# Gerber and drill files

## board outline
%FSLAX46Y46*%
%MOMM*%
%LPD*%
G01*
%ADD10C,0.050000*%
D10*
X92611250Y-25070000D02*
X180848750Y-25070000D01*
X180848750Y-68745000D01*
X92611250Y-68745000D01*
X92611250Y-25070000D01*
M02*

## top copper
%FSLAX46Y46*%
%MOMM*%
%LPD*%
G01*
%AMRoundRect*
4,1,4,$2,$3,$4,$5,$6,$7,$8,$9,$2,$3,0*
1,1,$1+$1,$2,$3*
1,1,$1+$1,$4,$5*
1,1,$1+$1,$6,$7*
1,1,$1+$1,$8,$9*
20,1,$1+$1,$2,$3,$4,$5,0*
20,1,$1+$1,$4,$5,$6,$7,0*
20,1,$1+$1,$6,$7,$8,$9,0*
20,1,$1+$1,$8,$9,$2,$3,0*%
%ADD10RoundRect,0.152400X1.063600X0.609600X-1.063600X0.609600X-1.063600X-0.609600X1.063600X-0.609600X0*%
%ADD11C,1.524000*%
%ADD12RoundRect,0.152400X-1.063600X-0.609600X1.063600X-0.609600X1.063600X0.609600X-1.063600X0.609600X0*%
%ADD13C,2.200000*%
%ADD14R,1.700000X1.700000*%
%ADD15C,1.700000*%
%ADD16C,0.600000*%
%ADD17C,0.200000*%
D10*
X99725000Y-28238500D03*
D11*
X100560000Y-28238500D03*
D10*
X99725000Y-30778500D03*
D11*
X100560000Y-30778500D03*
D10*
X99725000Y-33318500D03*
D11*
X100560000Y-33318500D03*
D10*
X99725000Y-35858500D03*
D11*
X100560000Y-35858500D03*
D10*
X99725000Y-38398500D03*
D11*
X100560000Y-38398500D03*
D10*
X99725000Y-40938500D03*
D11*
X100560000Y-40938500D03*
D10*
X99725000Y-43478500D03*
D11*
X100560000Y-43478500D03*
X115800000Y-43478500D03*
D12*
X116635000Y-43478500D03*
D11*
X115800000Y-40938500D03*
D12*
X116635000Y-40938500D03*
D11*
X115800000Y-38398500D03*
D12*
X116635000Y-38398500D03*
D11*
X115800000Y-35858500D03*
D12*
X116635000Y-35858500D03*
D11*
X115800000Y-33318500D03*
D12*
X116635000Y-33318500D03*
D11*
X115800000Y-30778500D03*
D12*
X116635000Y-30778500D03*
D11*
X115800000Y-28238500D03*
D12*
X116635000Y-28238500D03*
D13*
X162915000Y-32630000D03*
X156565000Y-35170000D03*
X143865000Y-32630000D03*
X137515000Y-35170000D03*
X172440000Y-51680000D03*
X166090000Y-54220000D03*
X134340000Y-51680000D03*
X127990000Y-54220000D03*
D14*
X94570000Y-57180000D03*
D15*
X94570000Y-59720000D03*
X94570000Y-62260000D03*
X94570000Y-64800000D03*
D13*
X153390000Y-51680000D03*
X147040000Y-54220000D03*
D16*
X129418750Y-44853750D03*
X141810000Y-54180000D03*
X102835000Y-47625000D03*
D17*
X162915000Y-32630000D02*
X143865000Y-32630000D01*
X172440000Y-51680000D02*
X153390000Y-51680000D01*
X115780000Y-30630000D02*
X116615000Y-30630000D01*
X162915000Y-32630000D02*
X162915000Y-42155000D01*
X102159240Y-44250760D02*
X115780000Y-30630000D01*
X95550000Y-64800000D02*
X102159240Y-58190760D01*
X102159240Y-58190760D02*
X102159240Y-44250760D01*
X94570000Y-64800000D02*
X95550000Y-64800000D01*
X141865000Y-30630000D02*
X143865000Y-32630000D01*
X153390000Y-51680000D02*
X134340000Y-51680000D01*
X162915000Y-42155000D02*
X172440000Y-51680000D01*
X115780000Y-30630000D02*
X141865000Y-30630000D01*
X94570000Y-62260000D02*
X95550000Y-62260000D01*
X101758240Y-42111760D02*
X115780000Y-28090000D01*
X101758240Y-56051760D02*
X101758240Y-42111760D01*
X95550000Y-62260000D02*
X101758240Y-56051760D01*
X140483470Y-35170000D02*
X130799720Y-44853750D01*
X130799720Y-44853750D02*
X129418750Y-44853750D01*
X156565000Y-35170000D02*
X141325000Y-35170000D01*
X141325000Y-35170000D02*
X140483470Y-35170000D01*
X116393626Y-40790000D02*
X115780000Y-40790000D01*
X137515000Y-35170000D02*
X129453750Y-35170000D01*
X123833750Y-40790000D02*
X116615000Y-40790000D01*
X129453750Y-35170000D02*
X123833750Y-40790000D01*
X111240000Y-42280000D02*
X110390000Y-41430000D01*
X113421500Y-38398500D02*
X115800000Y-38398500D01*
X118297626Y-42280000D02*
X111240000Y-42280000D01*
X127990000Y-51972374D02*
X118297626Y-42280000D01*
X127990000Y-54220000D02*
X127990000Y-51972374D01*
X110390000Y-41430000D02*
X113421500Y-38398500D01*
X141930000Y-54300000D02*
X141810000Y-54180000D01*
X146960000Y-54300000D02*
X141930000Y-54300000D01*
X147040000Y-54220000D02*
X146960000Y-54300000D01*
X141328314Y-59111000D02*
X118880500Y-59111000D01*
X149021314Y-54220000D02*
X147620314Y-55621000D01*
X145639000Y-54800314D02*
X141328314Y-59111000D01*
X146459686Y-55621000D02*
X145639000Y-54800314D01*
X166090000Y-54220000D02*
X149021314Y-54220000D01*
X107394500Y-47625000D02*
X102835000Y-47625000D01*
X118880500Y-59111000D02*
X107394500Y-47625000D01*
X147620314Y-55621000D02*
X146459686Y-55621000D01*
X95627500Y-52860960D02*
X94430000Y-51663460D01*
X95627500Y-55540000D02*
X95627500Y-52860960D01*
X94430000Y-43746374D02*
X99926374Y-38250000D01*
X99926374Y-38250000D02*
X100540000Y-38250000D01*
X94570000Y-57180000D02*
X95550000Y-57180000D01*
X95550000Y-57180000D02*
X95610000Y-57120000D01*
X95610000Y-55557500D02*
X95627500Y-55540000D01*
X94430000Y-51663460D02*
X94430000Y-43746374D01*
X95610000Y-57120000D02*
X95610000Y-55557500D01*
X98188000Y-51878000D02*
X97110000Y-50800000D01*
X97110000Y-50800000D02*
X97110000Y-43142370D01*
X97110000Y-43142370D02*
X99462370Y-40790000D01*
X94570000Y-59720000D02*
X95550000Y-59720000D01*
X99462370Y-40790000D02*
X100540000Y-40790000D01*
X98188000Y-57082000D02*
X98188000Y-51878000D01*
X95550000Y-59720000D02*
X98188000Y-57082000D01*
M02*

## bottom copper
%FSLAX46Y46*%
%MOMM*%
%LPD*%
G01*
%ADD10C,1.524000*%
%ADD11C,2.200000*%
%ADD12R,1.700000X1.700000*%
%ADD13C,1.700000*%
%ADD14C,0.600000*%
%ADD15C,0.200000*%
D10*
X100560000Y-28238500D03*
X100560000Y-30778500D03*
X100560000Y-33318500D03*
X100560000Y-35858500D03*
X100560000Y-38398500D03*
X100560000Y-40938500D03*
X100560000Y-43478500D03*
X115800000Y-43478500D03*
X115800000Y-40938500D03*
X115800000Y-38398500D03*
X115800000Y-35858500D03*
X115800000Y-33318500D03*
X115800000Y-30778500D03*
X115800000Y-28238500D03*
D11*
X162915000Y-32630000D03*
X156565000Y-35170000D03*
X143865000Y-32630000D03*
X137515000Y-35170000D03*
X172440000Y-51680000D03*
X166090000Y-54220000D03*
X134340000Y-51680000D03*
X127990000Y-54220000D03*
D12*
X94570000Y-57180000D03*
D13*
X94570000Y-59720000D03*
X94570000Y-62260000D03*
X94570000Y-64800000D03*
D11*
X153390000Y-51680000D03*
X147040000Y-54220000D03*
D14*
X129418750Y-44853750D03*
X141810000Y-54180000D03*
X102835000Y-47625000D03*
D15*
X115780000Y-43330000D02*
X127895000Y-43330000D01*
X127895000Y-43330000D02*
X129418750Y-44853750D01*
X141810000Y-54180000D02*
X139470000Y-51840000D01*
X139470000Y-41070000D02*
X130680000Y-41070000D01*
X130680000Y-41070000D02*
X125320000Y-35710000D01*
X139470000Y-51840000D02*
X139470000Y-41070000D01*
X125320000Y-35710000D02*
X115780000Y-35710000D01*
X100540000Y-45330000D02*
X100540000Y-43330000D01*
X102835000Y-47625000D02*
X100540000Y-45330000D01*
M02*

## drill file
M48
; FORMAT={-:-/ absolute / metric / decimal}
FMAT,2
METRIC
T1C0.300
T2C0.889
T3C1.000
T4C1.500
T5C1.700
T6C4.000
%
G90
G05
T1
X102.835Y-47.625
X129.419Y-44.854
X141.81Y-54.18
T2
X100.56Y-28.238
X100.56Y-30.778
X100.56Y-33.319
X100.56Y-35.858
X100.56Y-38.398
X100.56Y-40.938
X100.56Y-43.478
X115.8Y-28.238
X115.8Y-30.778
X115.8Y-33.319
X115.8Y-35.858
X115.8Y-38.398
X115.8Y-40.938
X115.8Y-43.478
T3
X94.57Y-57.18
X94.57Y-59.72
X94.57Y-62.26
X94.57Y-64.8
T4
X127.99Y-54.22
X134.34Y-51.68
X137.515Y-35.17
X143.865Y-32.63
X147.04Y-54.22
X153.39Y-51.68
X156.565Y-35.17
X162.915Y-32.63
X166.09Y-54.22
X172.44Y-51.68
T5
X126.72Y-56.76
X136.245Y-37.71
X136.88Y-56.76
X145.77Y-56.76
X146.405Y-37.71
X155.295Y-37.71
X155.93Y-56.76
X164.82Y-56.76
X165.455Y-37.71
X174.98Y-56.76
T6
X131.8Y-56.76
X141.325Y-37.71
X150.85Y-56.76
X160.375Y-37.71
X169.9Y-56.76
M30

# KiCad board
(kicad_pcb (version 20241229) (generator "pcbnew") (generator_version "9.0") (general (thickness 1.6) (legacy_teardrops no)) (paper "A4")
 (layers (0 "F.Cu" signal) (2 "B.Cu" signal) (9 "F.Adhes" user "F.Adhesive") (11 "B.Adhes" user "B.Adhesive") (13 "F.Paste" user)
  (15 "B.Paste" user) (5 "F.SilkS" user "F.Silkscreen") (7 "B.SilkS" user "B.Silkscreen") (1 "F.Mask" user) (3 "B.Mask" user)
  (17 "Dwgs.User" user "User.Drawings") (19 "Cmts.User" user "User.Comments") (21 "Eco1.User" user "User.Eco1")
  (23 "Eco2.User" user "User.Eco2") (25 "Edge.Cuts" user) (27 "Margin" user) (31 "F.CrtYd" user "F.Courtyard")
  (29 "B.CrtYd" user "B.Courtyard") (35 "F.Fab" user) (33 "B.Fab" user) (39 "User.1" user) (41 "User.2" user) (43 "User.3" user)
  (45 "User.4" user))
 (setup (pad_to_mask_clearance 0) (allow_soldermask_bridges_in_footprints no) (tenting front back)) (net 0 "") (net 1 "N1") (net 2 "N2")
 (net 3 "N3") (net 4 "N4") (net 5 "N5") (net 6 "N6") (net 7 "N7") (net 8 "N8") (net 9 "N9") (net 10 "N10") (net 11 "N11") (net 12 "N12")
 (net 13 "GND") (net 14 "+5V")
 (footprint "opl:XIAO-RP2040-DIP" (layer "F.Cu") (at 108.18 35.8585)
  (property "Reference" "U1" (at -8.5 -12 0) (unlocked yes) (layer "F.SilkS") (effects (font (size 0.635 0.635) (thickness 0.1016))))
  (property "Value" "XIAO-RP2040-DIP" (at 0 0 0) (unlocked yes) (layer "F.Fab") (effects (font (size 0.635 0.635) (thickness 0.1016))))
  (pad "1" smd roundrect (at -8.455 -7.62 180) (size 2.432 1.524) (layers "F.Cu" "F.Mask") (roundrect_rratio 0.1) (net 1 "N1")
   (thermal_bridge_angle 45))
  (pad "1" thru_hole circle (at -7.62 -7.62 180) (size 1.524 1.524) (drill 0.889) (layers "*.Cu" "*.Mask") (remove_unused_layers no)
   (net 1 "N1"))
  (pad "2" smd roundrect (at -8.455 -5.08 180) (size 2.432 1.524) (layers "F.Cu" "F.Mask") (roundrect_rratio 0.1) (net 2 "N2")
   (thermal_bridge_angle 45))
  (pad "2" thru_hole circle (at -7.62 -5.08 180) (size 1.524 1.524) (drill 0.889) (layers "*.Cu" "*.Mask") (remove_unused_layers no)
   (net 2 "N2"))
  (pad "3" smd roundrect (at -8.455 -2.54 180) (size 2.432 1.524) (layers "F.Cu" "F.Mask") (roundrect_rratio 0.1) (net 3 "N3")
   (thermal_bridge_angle 45))
  (pad "3" thru_hole circle (at -7.62 -2.54 180) (size 1.524 1.524) (drill 0.889) (layers "*.Cu" "*.Mask") (remove_unused_layers no)
   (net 3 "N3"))
  (pad "4" smd roundrect (at -8.455 0 180) (size 2.432 1.524) (layers "F.Cu" "F.Mask") (roundrect_rratio 0.1) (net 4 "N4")
   (thermal_bridge_angle 45))
  (pad "4" thru_hole circle (at -7.62 0 180) (size 1.524 1.524) (drill 0.889) (layers "*.Cu" "*.Mask") (remove_unused_layers no)
   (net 4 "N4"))
  (pad "5" smd roundrect (at -8.455 2.54 180) (size 2.432 1.524) (layers "F.Cu" "F.Mask") (roundrect_rratio 0.1) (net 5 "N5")
   (thermal_bridge_angle 45))
  (pad "5" thru_hole circle (at -7.62 2.54 180) (size 1.524 1.524) (drill 0.889) (layers "*.Cu" "*.Mask") (remove_unused_layers no)
   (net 5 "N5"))
  (pad "6" smd roundrect (at -8.455 5.08 180) (size 2.432 1.524) (layers "F.Cu" "F.Mask") (roundrect_rratio 0.1) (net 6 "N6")
   (thermal_bridge_angle 45))
  (pad "6" thru_hole circle (at -7.62 5.08 180) (size 1.524 1.524) (drill 0.889) (layers "*.Cu" "*.Mask") (remove_unused_layers no)
   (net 6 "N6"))
  (pad "7" smd roundrect (at -8.455 7.62 180) (size 2.432 1.524) (layers "F.Cu" "F.Mask") (roundrect_rratio 0.1) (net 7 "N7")
   (thermal_bridge_angle 45))
  (pad "7" thru_hole circle (at -7.62 7.62 180) (size 1.524 1.524) (drill 0.889) (layers "*.Cu" "*.Mask") (remove_unused_layers no)
   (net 7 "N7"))
  (pad "8" thru_hole circle (at 7.62 7.62) (size 1.524 1.524) (drill 0.889) (layers "*.Cu" "*.Mask") (remove_unused_layers no) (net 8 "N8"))
  (pad "8" smd roundrect (at 8.455 7.62) (size 2.432 1.524) (layers "F.Cu" "F.Mask") (roundrect_rratio 0.1) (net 8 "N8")
   (thermal_bridge_angle 45))
  (pad "9" thru_hole circle (at 7.62 5.08) (size 1.524 1.524) (drill 0.889) (layers "*.Cu" "*.Mask") (remove_unused_layers no) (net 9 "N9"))
  (pad "9" smd roundrect (at 8.455 5.08) (size 2.432 1.524) (layers "F.Cu" "F.Mask") (roundrect_rratio 0.1) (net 9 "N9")
   (thermal_bridge_angle 45))
  (pad "10" thru_hole circle (at 7.62 2.54) (size 1.524 1.524) (drill 0.889) (layers "*.Cu" "*.Mask") (remove_unused_layers no)
   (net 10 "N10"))
  (pad "10" smd roundrect (at 8.455 2.54) (size 2.432 1.524) (layers "F.Cu" "F.Mask") (roundrect_rratio 0.1) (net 10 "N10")
   (thermal_bridge_angle 45))
  (pad "11" thru_hole circle (at 7.62 0) (size 1.524 1.524) (drill 0.889) (layers "*.Cu" "*.Mask") (remove_unused_layers no) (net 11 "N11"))
  (pad "11" smd roundrect (at 8.455 0) (size 2.432 1.524) (layers "F.Cu" "F.Mask") (roundrect_rratio 0.1) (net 11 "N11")
   (thermal_bridge_angle 45))
  (pad "12" thru_hole circle (at 7.62 -2.54) (size 1.524 1.524) (drill 0.889) (layers "*.Cu" "*.Mask") (remove_unused_layers no)
   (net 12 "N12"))
  (pad "12" smd roundrect (at 8.455 -2.54) (size 2.432 1.524) (layers "F.Cu" "F.Mask") (roundrect_rratio 0.1) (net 12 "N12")
   (thermal_bridge_angle 45))
  (pad "13" thru_hole circle (at 7.62 -5.08) (size 1.524 1.524) (drill 0.889) (layers "*.Cu" "*.Mask") (remove_unused_layers no)
   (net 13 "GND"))
  (pad "13" smd roundrect (at 8.455 -5.08) (size 2.432 1.524) (layers "F.Cu" "F.Mask") (roundrect_rratio 0.1) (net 13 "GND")
   (thermal_bridge_angle 45))
  (pad "14" thru_hole circle (at 7.62 -7.62) (size 1.524 1.524) (drill 0.889) (layers "*.Cu" "*.Mask") (remove_unused_layers no)
   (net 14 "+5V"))
  (pad "14" smd roundrect (at 8.455 -7.62) (size 2.432 1.524) (layers "F.Cu" "F.Mask") (roundrect_rratio 0.1) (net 14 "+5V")
   (thermal_bridge_angle 45)))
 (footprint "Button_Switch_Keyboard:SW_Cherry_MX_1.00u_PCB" (layer "F.Cu") (at 162.915 32.63)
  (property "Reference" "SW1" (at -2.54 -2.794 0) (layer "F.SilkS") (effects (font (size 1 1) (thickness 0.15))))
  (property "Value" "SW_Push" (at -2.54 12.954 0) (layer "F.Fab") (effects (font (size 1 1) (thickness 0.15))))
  (pad "" np_thru_hole circle (at -7.62 5.08) (size 1.7 1.7) (drill 1.7) (layers "*.Cu" "*.Mask"))
  (pad "" np_thru_hole circle (at -2.54 5.08) (size 4 4) (drill 4) (layers "*.Cu" "*.Mask"))
  (pad "" np_thru_hole circle (at 2.54 5.08) (size 1.7 1.7) (drill 1.7) (layers "*.Cu" "*.Mask"))
  (pad "1" thru_hole circle (at 0 0) (size 2.2 2.2) (drill 1.5) (layers "*.Cu" "*.Mask") (remove_unused_layers no) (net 13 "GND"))
  (pad "2" thru_hole circle (at -6.35 2.54) (size 2.2 2.2) (drill 1.5) (layers "*.Cu" "*.Mask") (remove_unused_layers no) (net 8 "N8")))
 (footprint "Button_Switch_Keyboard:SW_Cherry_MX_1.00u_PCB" (layer "F.Cu") (at 143.865 32.63)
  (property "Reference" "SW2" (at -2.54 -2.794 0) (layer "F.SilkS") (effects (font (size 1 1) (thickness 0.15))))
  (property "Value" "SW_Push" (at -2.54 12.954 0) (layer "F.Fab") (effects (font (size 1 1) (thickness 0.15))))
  (pad "" np_thru_hole circle (at -7.62 5.08) (size 1.7 1.7) (drill 1.7) (layers "*.Cu" "*.Mask"))
  (pad "" np_thru_hole circle (at -2.54 5.08) (size 4 4) (drill 4) (layers "*.Cu" "*.Mask"))
  (pad "" np_thru_hole circle (at 2.54 5.08) (size 1.7 1.7) (drill 1.7) (layers "*.Cu" "*.Mask"))
  (pad "1" thru_hole circle (at 0 0) (size 2.2 2.2) (drill 1.5) (layers "*.Cu" "*.Mask") (remove_unused_layers no) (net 13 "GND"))
  (pad "2" thru_hole circle (at -6.35 2.54) (size 2.2 2.2) (drill 1.5) (layers "*.Cu" "*.Mask") (remove_unused_layers no) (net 9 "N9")))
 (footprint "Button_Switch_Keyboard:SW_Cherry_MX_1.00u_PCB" (layer "F.Cu") (at 172.44 51.68)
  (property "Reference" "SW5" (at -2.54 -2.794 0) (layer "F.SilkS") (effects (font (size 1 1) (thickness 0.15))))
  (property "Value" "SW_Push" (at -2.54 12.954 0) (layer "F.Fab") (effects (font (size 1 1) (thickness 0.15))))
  (pad "" np_thru_hole circle (at -7.62 5.08) (size 1.7 1.7) (drill 1.7) (layers "*.Cu" "*.Mask"))
  (pad "" np_thru_hole circle (at -2.54 5.08) (size 4 4) (drill 4) (layers "*.Cu" "*.Mask"))
  (pad "" np_thru_hole circle (at 2.54 5.08) (size 1.7 1.7) (drill 1.7) (layers "*.Cu" "*.Mask"))
  (pad "1" thru_hole circle (at 0 0) (size 2.2 2.2) (drill 1.5) (layers "*.Cu" "*.Mask") (remove_unused_layers no) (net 13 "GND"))
  (pad "2" thru_hole circle (at -6.35 2.54) (size 2.2 2.2) (drill 1.5) (layers "*.Cu" "*.Mask") (remove_unused_layers no) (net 7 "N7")))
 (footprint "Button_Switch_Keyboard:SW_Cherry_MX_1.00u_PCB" (layer "F.Cu") (at 134.34 51.68)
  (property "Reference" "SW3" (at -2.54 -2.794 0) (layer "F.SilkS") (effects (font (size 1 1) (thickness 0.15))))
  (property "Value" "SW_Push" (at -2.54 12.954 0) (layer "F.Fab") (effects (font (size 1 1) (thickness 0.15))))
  (pad "" np_thru_hole circle (at -7.62 5.08) (size 1.7 1.7) (drill 1.7) (layers "*.Cu" "*.Mask"))
  (pad "" np_thru_hole circle (at -2.54 5.08) (size 4 4) (drill 4) (layers "*.Cu" "*.Mask"))
  (pad "" np_thru_hole circle (at 2.54 5.08) (size 1.7 1.7) (drill 1.7) (layers "*.Cu" "*.Mask"))
  (pad "1" thru_hole circle (at 0 0) (size 2.2 2.2) (drill 1.5) (layers "*.Cu" "*.Mask") (remove_unused_layers no) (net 13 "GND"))
  (pad "2" thru_hole circle (at -6.35 2.54) (size 2.2 2.2) (drill 1.5) (layers "*.Cu" "*.Mask") (remove_unused_layers no) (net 10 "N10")))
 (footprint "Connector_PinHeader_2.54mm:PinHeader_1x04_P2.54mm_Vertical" (layer "F.Cu") (at 94.57 57.18)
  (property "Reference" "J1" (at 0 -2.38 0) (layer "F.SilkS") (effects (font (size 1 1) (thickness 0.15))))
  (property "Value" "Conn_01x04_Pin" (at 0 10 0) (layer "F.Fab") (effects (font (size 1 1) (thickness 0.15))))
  (pad "1" thru_hole rect (at 0 0) (size 1.7 1.7) (drill 1) (layers "*.Cu" "*.Mask") (remove_unused_layers no) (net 5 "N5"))
  (pad "2" thru_hole circle (at 0 2.54) (size 1.7 1.7) (drill 1) (layers "*.Cu" "*.Mask") (remove_unused_layers no) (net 6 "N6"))
  (pad "3" thru_hole circle (at 0 5.08) (size 1.7 1.7) (drill 1) (layers "*.Cu" "*.Mask") (remove_unused_layers no) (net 14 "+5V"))
  (pad "4" thru_hole circle (at 0 7.62) (size 1.7 1.7) (drill 1) (layers "*.Cu" "*.Mask") (remove_unused_layers no) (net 13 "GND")))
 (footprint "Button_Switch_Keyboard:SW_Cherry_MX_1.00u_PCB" (layer "F.Cu") (at 153.39 51.68)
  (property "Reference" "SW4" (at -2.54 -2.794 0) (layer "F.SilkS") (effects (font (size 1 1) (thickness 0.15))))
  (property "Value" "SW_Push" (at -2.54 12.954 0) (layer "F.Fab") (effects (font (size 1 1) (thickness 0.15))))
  (pad "" np_thru_hole circle (at -7.62 5.08) (size 1.7 1.7) (drill 1.7) (layers "*.Cu" "*.Mask"))
  (pad "" np_thru_hole circle (at -2.54 5.08) (size 4 4) (drill 4) (layers "*.Cu" "*.Mask"))
  (pad "" np_thru_hole circle (at 2.54 5.08) (size 1.7 1.7) (drill 1.7) (layers "*.Cu" "*.Mask"))
  (pad "1" thru_hole circle (at 0 0) (size 2.2 2.2) (drill 1.5) (layers "*.Cu" "*.Mask") (remove_unused_layers no) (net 13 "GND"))
  (pad "2" thru_hole circle (at -6.35 2.54) (size 2.2 2.2) (drill 1.5) (layers "*.Cu" "*.Mask") (remove_unused_layers no) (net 11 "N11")))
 (gr_rect (start 92.61125 25.07) (end 180.84875 68.745) (stroke (width 0.05) (type default)) (fill no) (layer "Edge.Cuts"))
 (segment (start 162.915 32.63) (end 143.865 32.63) (width 0.2) (layer "F.Cu") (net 13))
 (segment (start 172.44 51.68) (end 153.39 51.68) (width 0.2) (layer "F.Cu") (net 13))
 (segment (start 115.78 30.63) (end 116.615 30.63) (width 0.2) (layer "F.Cu") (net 13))
 (segment (start 162.915 32.63) (end 162.915 42.155) (width 0.2) (layer "F.Cu") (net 13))
 (segment (start 102.15924 44.25076) (end 115.78 30.63) (width 0.2) (layer "F.Cu") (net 13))
 (segment (start 95.55 64.8) (end 102.15924 58.19076) (width 0.2) (layer "F.Cu") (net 13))
 (segment (start 102.15924 58.19076) (end 102.15924 44.25076) (width 0.2) (layer "F.Cu") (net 13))
 (segment (start 94.57 64.8) (end 95.55 64.8) (width 0.2) (layer "F.Cu") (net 13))
 (segment (start 141.865 30.63) (end 143.865 32.63) (width 0.2) (layer "F.Cu") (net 13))
 (segment (start 153.39 51.68) (end 134.34 51.68) (width 0.2) (layer "F.Cu") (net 13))
 (segment (start 162.915 42.155) (end 172.44 51.68) (width 0.2) (layer "F.Cu") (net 13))
 (segment (start 115.78 30.63) (end 141.865 30.63) (width 0.2) (layer "F.Cu") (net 13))
 (segment (start 94.57 62.26) (end 95.55 62.26) (width 0.2) (layer "F.Cu") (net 14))
 (segment (start 101.75824 42.11176) (end 115.78 28.09) (width 0.2) (layer "F.Cu") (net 14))
 (segment (start 101.75824 56.05176) (end 101.75824 42.11176) (width 0.2) (layer "F.Cu") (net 14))
 (segment (start 95.55 62.26) (end 101.75824 56.05176) (width 0.2) (layer "F.Cu") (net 14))
 (segment (start 140.48347 35.17) (end 130.79972 44.85375) (width 0.2) (layer "F.Cu") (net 8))
 (segment (start 130.79972 44.85375) (end 129.41875 44.85375) (width 0.2) (layer "F.Cu") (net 8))
 (segment (start 156.565 35.17) (end 141.325 35.17) (width 0.2) (layer "F.Cu") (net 8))
 (segment (start 141.325 35.17) (end 140.48347 35.17) (width 0.2) (layer "F.Cu") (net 8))
 (via (at 129.41875 44.85375) (size 0.6) (drill 0.3) (layers "F.Cu" "B.Cu") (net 8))
 (segment (start 115.78 43.33) (end 127.895 43.33) (width 0.2) (layer "B.Cu") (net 8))
 (segment (start 127.895 43.33) (end 129.41875 44.85375) (width 0.2) (layer "B.Cu") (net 8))
 (segment (start 116.393626 40.79) (end 115.78 40.79) (width 0.2) (layer "F.Cu") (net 9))
 (segment (start 137.515 35.17) (end 129.45375 35.17) (width 0.2) (layer "F.Cu") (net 9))
 (segment (start 123.83375 40.79) (end 116.615 40.79) (width 0.2) (layer "F.Cu") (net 9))
 (segment (start 129.45375 35.17) (end 123.83375 40.79) (width 0.2) (layer "F.Cu") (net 9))
 (segment (start 111.24 42.28) (end 110.39 41.43) (width 0.2) (layer "F.Cu") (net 10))
 (segment (start 113.4215 38.3985) (end 115.8 38.3985) (width 0.2) (layer "F.Cu") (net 10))
 (segment (start 118.297626 42.28) (end 111.24 42.28) (width 0.2) (layer "F.Cu") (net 10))
 (segment (start 127.99 51.972374) (end 118.297626 42.28) (width 0.2) (layer "F.Cu") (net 10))
 (segment (start 127.99 54.22) (end 127.99 51.972374) (width 0.2) (layer "F.Cu") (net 10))
 (segment (start 110.39 41.43) (end 113.4215 38.3985) (width 0.2) (layer "F.Cu") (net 10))
 (segment (start 141.93 54.3) (end 141.81 54.18) (width 0.2) (layer "F.Cu") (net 11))
 (segment (start 146.96 54.3) (end 141.93 54.3) (width 0.2) (layer "F.Cu") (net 11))
 (segment (start 147.04 54.22) (end 146.96 54.3) (width 0.2) (layer "F.Cu") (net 11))
 (via (at 141.81 54.18) (size 0.6) (drill 0.3) (layers "F.Cu" "B.Cu") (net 11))
 (segment (start 141.81 54.18) (end 139.47 51.84) (width 0.2) (layer "B.Cu") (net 11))
 (segment (start 139.47 41.07) (end 130.68 41.07) (width 0.2) (layer "B.Cu") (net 11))
 (segment (start 130.68 41.07) (end 125.32 35.71) (width 0.2) (layer "B.Cu") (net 11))
 (segment (start 139.47 51.84) (end 139.47 41.07) (width 0.2) (layer "B.Cu") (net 11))
 (segment (start 125.32 35.71) (end 115.78 35.71) (width 0.2) (layer "B.Cu") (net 11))
 (segment (start 141.328314 59.111) (end 118.8805 59.111) (width 0.2) (layer "F.Cu") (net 7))
 (segment (start 149.021314 54.22) (end 147.620314 55.621) (width 0.2) (layer "F.Cu") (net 7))
 (segment (start 145.639 54.800314) (end 141.328314 59.111) (width 0.2) (layer "F.Cu") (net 7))
 (segment (start 146.459686 55.621) (end 145.639 54.800314) (width 0.2) (layer "F.Cu") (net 7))
 (segment (start 166.09 54.22) (end 149.021314 54.22) (width 0.2) (layer "F.Cu") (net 7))
 (segment (start 107.3945 47.625) (end 102.835 47.625) (width 0.2) (layer "F.Cu") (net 7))
 (segment (start 118.8805 59.111) (end 107.3945 47.625) (width 0.2) (layer "F.Cu") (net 7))
 (segment (start 147.620314 55.621) (end 146.459686 55.621) (width 0.2) (layer "F.Cu") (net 7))
 (via (at 102.835 47.625) (size 0.6) (drill 0.3) (layers "F.Cu" "B.Cu") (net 7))
 (segment (start 100.54 45.33) (end 100.54 43.33) (width 0.2) (layer "B.Cu") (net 7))
 (segment (start 102.835 47.625) (end 100.54 45.33) (width 0.2) (layer "B.Cu") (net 7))
 (segment (start 95.6275 52.86096) (end 94.43 51.66346) (width 0.2) (layer "F.Cu") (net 5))
 (segment (start 95.6275 55.54) (end 95.6275 52.86096) (width 0.2) (layer "F.Cu") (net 5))
 (segment (start 94.43 43.746374) (end 99.926374 38.25) (width 0.2) (layer "F.Cu") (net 5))
 (segment (start 99.926374 38.25) (end 100.54 38.25) (width 0.2) (layer "F.Cu") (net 5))
 (segment (start 94.57 57.18) (end 95.55 57.18) (width 0.2) (layer "F.Cu") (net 5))
 (segment (start 95.55 57.18) (end 95.61 57.12) (width 0.2) (layer "F.Cu") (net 5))
 (segment (start 95.61 55.5575) (end 95.6275 55.54) (width 0.2) (layer "F.Cu") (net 5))
 (segment (start 94.43 51.66346) (end 94.43 43.746374) (width 0.2) (layer "F.Cu") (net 5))
 (segment (start 95.61 57.12) (end 95.61 55.5575) (width 0.2) (layer "F.Cu") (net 5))
 (segment (start 98.188 51.878) (end 97.11 50.8) (width 0.2) (layer "F.Cu") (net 6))
 (segment (start 97.11 50.8) (end 97.11 43.14237) (width 0.2) (layer "F.Cu") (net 6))
 (segment (start 97.11 43.14237) (end 99.46237 40.79) (width 0.2) (layer "F.Cu") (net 6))
 (segment (start 94.57 59.72) (end 95.55 59.72) (width 0.2) (layer "F.Cu") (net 6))
 (segment (start 99.46237 40.79) (end 100.54 40.79) (width 0.2) (layer "F.Cu") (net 6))
 (segment (start 98.188 57.082) (end 98.188 51.878) (width 0.2) (layer "F.Cu") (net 6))
 (segment (start 95.55 59.72) (end 98.188 57.082) (width 0.2) (layer "F.Cu") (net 6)))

